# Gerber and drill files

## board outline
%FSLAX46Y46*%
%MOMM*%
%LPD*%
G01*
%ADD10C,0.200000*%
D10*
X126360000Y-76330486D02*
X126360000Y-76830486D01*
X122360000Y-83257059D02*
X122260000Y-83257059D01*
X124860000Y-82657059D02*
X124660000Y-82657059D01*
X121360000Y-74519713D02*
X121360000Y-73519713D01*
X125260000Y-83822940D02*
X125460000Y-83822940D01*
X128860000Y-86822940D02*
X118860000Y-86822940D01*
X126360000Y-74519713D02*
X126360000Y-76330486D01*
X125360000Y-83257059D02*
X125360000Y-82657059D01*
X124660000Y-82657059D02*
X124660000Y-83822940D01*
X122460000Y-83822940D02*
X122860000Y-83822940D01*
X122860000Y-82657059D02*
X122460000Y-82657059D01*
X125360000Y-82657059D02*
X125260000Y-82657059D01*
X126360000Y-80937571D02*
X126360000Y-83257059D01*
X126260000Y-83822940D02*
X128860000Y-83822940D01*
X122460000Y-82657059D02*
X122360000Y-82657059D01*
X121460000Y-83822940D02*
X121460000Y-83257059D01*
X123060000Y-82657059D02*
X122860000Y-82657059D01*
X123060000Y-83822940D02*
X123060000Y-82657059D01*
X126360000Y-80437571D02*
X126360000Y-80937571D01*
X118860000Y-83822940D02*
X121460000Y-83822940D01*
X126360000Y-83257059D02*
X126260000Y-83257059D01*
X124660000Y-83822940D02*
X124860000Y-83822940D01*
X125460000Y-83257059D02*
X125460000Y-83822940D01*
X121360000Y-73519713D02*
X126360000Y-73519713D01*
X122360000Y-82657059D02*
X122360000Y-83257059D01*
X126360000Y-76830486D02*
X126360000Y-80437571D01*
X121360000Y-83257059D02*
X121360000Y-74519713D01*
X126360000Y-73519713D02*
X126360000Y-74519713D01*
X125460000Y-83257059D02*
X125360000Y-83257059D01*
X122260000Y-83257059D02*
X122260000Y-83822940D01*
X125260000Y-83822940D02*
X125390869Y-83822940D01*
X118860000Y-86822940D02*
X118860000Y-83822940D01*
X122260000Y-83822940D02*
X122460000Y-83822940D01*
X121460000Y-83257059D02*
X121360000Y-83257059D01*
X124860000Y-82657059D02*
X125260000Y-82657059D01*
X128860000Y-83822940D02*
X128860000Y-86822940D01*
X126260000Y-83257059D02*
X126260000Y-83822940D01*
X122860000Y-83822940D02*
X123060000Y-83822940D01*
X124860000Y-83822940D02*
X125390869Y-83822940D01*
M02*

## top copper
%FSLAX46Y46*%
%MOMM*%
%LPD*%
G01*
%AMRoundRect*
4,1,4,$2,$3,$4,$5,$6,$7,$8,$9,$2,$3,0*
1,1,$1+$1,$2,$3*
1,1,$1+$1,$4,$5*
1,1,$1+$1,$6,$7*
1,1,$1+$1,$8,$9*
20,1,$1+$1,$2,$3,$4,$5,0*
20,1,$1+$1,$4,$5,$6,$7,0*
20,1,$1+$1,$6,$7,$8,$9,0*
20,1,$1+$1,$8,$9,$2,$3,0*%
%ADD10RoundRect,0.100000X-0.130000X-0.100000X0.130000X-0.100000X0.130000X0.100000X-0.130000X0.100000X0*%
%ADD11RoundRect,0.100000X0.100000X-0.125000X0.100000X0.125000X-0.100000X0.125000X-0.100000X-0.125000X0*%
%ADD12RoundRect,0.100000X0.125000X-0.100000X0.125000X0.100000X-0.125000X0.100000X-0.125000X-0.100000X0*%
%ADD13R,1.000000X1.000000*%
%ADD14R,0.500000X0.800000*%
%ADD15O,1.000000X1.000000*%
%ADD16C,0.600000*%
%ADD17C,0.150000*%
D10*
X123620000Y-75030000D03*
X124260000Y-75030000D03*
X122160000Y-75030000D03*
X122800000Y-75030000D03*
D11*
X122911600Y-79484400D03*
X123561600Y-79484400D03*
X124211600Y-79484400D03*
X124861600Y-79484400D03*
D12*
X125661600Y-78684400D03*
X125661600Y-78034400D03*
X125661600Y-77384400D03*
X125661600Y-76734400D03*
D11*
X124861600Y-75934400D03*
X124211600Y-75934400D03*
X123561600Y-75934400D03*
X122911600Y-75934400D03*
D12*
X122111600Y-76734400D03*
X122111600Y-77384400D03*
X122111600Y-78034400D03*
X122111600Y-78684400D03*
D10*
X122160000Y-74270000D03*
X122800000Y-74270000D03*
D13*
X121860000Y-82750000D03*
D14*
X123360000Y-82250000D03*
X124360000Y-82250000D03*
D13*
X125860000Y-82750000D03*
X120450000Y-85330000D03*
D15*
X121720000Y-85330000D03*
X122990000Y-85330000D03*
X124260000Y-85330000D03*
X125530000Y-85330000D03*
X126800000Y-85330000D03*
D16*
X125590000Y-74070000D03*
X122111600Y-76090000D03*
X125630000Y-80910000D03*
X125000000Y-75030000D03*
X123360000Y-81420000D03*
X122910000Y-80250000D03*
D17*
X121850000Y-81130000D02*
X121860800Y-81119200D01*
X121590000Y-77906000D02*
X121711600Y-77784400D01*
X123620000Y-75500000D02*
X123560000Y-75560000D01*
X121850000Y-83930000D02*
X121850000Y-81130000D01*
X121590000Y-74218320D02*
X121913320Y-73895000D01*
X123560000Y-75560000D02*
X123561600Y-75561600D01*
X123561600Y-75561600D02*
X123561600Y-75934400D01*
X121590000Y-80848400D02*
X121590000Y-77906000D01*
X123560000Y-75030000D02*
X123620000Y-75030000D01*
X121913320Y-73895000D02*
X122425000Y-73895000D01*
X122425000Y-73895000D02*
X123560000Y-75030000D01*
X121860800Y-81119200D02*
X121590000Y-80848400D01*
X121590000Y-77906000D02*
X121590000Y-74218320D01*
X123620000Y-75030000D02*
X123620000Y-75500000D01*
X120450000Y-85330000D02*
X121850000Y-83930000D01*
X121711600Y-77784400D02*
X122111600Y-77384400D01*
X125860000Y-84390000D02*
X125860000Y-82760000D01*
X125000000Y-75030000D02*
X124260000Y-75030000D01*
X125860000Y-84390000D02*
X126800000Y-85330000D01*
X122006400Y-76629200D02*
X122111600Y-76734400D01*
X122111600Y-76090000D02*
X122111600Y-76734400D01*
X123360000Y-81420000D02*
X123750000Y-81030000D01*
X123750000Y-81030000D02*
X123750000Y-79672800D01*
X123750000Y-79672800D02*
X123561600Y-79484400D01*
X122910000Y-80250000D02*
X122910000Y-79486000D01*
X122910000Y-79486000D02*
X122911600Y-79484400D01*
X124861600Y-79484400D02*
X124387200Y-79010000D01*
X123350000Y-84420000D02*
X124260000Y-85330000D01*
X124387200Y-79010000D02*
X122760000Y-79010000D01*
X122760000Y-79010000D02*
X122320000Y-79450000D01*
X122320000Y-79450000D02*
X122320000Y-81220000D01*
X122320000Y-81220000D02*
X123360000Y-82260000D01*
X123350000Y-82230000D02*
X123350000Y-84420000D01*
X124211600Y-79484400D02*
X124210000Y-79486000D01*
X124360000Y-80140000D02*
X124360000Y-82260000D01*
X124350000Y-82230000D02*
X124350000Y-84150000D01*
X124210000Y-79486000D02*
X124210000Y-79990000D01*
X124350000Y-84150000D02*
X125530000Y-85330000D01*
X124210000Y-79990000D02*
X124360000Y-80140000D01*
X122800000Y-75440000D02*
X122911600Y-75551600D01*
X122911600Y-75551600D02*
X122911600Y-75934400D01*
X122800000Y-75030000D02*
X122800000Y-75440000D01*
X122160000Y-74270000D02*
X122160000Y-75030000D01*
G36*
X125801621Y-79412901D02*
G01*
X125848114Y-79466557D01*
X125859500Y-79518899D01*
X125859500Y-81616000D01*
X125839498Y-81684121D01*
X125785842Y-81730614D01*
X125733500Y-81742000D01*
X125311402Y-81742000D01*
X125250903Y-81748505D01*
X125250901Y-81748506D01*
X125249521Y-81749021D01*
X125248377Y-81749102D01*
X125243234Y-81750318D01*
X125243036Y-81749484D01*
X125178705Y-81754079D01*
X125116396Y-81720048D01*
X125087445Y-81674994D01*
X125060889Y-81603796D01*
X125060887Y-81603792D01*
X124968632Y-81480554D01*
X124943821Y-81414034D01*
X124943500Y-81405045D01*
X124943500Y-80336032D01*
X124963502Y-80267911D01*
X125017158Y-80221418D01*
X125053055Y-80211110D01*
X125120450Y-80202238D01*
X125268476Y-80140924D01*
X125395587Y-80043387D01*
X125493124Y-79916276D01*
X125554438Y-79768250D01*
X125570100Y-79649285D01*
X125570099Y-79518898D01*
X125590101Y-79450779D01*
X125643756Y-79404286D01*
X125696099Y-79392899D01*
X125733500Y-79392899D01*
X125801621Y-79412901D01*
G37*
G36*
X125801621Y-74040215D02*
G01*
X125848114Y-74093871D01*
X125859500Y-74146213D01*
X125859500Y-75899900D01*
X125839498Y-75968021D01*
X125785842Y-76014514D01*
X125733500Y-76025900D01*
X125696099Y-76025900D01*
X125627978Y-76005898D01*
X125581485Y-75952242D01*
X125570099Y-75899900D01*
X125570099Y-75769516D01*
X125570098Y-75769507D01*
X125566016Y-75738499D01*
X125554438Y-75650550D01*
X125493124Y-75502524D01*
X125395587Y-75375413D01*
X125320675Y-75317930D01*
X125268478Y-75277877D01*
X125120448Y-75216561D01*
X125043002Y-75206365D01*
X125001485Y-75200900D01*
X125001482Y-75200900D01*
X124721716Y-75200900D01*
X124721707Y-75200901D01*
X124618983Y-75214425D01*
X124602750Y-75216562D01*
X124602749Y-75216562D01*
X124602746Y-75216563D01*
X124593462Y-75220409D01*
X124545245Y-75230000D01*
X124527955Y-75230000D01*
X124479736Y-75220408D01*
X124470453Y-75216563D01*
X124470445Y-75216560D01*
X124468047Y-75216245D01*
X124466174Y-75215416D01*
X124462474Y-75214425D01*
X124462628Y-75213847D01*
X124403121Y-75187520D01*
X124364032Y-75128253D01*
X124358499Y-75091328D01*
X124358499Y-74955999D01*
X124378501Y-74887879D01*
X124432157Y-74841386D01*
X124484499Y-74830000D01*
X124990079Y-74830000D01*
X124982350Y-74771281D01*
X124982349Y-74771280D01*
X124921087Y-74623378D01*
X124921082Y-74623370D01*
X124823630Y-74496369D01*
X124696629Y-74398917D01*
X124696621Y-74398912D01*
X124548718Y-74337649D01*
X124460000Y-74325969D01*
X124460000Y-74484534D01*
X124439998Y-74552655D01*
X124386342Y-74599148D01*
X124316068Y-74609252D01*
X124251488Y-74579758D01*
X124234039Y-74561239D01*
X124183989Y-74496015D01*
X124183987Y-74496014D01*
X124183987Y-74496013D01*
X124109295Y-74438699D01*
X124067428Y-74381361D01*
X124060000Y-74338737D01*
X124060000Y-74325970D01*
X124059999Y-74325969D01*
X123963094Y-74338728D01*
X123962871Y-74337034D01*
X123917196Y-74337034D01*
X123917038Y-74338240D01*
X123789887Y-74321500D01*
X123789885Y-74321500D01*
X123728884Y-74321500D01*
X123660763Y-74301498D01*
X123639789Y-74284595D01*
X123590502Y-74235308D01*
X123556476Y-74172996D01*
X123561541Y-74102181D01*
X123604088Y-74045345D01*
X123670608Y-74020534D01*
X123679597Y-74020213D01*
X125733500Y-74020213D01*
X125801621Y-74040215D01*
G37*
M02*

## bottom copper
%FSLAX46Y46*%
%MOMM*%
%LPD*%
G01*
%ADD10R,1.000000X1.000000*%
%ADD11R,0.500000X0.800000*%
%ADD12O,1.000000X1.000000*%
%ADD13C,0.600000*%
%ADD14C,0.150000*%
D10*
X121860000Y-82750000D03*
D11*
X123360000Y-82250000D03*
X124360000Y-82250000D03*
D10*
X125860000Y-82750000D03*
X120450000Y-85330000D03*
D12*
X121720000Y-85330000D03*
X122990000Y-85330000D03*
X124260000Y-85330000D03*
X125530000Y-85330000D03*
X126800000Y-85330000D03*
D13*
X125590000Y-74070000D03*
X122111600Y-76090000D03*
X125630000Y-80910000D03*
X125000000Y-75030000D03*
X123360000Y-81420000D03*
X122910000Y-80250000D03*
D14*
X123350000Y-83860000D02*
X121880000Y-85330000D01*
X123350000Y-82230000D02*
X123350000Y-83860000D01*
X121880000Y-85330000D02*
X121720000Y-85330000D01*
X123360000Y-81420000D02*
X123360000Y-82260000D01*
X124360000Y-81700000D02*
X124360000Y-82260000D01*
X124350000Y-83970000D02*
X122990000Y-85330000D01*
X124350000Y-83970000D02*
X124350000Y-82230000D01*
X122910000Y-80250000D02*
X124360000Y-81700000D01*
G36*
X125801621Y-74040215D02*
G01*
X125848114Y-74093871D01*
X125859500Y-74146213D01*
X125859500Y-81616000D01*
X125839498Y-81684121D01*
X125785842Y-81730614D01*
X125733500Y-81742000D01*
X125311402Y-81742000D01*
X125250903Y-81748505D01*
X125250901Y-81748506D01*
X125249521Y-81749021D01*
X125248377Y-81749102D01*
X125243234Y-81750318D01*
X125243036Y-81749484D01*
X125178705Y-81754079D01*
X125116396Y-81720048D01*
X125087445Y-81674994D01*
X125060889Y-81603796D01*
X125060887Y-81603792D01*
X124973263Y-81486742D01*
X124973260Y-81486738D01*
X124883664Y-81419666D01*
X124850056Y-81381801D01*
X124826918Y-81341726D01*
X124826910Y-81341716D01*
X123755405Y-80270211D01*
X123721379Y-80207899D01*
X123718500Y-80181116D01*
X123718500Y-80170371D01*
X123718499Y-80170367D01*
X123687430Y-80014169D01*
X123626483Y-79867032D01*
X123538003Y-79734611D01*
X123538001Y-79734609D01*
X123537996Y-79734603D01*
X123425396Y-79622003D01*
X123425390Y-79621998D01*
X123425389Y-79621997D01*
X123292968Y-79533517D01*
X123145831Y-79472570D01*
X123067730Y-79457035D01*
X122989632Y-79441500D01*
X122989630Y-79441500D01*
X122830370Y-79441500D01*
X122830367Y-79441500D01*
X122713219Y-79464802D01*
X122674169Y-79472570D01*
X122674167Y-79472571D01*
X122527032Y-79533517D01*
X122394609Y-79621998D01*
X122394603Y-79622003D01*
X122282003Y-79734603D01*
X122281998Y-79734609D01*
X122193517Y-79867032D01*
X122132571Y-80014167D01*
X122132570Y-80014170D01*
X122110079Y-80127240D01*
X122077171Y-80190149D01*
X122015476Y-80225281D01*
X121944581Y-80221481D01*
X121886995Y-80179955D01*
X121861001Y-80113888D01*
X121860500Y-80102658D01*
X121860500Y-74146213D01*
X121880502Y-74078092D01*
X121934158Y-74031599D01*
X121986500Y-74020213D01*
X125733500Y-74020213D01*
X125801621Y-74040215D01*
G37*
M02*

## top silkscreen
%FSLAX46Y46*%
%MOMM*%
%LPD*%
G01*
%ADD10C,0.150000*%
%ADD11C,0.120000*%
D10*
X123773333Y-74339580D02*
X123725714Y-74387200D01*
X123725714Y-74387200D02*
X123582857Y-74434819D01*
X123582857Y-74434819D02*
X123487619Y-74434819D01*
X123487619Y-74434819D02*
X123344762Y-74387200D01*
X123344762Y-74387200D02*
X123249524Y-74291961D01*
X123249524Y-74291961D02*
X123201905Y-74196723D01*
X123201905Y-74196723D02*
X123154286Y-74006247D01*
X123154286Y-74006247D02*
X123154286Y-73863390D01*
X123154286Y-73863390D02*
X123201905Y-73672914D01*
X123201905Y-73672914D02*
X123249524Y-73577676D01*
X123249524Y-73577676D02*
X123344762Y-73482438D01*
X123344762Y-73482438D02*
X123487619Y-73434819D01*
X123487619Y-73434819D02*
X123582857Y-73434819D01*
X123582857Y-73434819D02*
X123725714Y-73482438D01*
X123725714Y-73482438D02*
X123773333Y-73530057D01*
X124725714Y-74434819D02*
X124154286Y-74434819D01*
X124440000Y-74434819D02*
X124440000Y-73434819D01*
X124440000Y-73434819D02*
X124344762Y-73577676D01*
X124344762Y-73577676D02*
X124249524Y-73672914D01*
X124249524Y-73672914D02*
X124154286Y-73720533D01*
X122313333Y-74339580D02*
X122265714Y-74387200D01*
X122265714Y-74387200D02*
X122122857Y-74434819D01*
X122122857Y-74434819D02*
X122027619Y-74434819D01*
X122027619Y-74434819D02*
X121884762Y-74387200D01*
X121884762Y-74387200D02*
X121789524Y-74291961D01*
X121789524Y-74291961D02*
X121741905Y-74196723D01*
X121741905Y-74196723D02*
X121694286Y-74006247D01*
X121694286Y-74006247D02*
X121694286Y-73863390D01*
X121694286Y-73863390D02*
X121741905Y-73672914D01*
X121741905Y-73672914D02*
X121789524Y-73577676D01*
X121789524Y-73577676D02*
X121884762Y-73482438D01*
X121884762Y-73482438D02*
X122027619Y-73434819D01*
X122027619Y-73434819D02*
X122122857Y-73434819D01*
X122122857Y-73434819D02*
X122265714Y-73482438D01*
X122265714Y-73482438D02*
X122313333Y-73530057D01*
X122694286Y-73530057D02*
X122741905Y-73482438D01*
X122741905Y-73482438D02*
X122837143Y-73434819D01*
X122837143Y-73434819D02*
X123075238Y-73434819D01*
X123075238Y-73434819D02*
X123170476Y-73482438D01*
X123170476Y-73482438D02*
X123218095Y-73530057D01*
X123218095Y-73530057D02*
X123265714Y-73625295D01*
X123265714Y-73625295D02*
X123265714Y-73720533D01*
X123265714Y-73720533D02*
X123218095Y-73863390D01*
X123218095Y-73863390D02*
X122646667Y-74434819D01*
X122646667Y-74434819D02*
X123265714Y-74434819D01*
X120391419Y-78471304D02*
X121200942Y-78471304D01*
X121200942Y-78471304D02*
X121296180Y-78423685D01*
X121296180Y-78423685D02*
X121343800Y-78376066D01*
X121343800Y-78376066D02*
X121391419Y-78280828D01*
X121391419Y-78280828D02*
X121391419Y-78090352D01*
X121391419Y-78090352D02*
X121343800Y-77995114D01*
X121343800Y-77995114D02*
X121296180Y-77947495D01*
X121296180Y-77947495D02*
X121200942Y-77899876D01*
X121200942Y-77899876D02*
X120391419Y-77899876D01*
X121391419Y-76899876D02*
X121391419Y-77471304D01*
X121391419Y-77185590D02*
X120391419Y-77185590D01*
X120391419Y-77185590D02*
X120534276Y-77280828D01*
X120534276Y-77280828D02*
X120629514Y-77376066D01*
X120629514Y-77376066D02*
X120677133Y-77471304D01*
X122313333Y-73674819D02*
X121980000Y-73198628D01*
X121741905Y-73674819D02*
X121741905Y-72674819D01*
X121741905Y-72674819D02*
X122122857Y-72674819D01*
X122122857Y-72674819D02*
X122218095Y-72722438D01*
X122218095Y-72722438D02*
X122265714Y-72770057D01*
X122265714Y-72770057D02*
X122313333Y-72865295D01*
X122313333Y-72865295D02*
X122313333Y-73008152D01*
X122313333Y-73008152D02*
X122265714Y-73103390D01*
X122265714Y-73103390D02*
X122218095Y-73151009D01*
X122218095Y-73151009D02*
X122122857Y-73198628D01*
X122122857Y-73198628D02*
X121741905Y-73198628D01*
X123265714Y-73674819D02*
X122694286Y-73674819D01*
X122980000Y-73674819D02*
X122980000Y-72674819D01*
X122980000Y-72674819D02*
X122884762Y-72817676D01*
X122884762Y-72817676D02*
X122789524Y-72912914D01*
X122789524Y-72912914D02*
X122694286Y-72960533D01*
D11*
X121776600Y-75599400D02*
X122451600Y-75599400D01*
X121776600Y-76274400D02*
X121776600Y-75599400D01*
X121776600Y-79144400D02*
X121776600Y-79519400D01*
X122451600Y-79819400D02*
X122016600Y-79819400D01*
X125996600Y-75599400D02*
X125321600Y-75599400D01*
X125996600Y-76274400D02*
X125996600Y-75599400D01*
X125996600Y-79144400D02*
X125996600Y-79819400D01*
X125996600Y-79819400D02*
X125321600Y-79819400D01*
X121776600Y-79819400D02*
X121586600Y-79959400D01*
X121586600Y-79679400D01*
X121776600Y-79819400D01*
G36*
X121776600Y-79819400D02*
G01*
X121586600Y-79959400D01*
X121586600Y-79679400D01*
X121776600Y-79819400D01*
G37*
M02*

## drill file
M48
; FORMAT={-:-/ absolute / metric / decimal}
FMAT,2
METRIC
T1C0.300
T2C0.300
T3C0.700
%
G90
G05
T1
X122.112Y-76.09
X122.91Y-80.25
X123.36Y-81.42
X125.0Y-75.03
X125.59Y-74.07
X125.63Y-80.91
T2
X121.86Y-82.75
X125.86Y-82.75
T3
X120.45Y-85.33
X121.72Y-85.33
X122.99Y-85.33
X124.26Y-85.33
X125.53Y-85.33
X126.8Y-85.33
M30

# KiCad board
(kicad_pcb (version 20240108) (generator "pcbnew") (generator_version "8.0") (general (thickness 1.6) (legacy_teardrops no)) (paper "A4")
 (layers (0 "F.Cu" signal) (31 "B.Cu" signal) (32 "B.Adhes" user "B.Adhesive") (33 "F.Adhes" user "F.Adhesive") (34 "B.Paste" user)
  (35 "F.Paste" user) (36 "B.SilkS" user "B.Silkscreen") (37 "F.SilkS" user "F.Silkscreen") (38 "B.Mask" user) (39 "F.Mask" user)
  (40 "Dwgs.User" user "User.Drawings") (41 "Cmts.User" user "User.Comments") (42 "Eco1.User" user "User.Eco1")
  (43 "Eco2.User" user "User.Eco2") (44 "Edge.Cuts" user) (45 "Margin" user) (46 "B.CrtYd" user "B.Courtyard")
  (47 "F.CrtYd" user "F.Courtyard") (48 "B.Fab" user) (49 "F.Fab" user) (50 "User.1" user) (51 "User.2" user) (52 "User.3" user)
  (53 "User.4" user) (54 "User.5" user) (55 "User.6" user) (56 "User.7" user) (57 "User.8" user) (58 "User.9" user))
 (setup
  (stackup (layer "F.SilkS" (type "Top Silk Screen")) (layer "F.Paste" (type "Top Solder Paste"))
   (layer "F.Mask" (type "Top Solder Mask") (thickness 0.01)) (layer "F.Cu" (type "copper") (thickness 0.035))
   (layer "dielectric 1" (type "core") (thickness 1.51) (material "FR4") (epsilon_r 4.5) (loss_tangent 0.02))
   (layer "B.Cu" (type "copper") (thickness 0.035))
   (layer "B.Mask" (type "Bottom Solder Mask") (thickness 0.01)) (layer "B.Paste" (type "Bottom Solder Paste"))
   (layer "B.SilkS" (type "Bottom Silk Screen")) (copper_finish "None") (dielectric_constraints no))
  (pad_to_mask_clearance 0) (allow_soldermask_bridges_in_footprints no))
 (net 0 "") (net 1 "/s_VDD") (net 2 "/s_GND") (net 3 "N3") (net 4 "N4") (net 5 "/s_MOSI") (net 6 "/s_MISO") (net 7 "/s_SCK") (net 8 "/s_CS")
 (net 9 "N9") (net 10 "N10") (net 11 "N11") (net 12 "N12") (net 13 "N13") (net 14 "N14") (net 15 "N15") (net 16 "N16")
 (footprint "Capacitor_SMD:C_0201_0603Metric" (layer "F.Cu") (at 123.94 75.03)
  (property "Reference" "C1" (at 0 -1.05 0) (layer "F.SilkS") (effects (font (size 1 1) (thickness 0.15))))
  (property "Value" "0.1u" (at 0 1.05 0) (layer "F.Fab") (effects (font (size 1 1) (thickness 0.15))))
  (pad "" smd roundrect (at -0.345 0) (size 0.318 0.36) (layers "F.Paste") (roundrect_rratio 0.25))
  (pad "" smd roundrect (at 0.345 0) (size 0.318 0.36) (layers "F.Paste") (roundrect_rratio 0.25))
  (pad "1" smd roundrect (at -0.32 0) (size 0.46 0.4) (layers "F.Cu" "F.Mask") (roundrect_rratio 0.25) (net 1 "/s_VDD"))
  (pad "2" smd roundrect (at 0.32 0) (size 0.46 0.4) (layers "F.Cu" "F.Mask") (roundrect_rratio 0.25) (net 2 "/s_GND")))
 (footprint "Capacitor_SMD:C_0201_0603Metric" (layer "F.Cu") (at 122.48 75.03)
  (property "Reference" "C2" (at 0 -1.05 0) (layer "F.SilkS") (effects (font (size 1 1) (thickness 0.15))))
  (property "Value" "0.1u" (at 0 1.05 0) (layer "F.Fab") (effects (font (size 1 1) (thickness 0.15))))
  (pad "" smd roundrect (at -0.345 0) (size 0.318 0.36) (layers "F.Paste") (roundrect_rratio 0.25))
  (pad "" smd roundrect (at 0.345 0) (size 0.318 0.36) (layers "F.Paste") (roundrect_rratio 0.25))
  (pad "1" smd roundrect (at -0.32 0) (size 0.46 0.4) (layers "F.Cu" "F.Mask") (roundrect_rratio 0.25) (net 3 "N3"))
  (pad "2" smd roundrect (at 0.32 0) (size 0.46 0.4) (layers "F.Cu" "F.Mask") (roundrect_rratio 0.25) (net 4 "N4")))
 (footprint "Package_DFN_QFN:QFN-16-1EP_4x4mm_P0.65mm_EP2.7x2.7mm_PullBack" (layer "F.Cu") (at 123.8866 77.7094 90)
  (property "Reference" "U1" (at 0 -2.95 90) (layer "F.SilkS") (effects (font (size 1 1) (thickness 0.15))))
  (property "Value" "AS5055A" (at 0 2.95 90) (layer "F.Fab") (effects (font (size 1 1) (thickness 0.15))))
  (fp_line (start 2.11 -2.11) (end 2.11 -1.435) (stroke (width 0.12) (type solid)) (layer "F.SilkS"))
  (fp_line (start 1.435 -2.11) (end 2.11 -2.11) (stroke (width 0.12) (type solid)) (layer "F.SilkS"))
  (fp_line (start -1.435 -2.11) (end -1.81 -2.11) (stroke (width 0.12) (type solid)) (layer "F.SilkS"))
  (fp_line (start -2.11 -1.435) (end -2.11 -1.87) (stroke (width 0.12) (type solid)) (layer "F.SilkS"))
  (fp_line (start 2.11 2.11) (end 2.11 1.435) (stroke (width 0.12) (type solid)) (layer "F.SilkS"))
  (fp_line (start 1.435 2.11) (end 2.11 2.11) (stroke (width 0.12) (type solid)) (layer "F.SilkS"))
  (fp_line (start -1.435 2.11) (end -2.11 2.11) (stroke (width 0.12) (type solid)) (layer "F.SilkS"))
  (fp_line (start -2.11 2.11) (end -2.11 1.435) (stroke (width 0.12) (type solid)) (layer "F.SilkS"))
  (fp_poly
   (pts (xy -2.11 -2.11) (xy -2.25 -2.3) (xy -1.97 -2.3) (xy -2.11 -2.11)) (stroke (width 0.12) (type solid)) (fill solid) (layer "F.SilkS"))
  (pad "1" smd roundrect (at -1.775 -0.975 90) (size 0.45 0.4) (layers "F.Cu" "F.Paste" "F.Mask") (roundrect_rratio 0.25) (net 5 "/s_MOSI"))
  (pad "2" smd roundrect (at -1.775 -0.325 90) (size 0.45 0.4) (layers "F.Cu" "F.Paste" "F.Mask") (roundrect_rratio 0.25) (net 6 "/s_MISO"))
  (pad "3" smd roundrect (at -1.775 0.325 90) (size 0.45 0.4) (layers "F.Cu" "F.Paste" "F.Mask") (roundrect_rratio 0.25) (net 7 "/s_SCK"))
  (pad "4" smd roundrect (at -1.775 0.975 90) (size 0.45 0.4) (layers "F.Cu" "F.Paste" "F.Mask") (roundrect_rratio 0.25) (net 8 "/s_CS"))
  (pad "5" smd roundrect (at -0.975 1.775 90) (size 0.4 0.45) (layers "F.Cu" "F.Paste" "F.Mask") (roundrect_rratio 0.25) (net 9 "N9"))
  (pad "6" smd roundrect (at -0.325 1.775 90) (size 0.4 0.45) (layers "F.Cu" "F.Paste" "F.Mask") (roundrect_rratio 0.25) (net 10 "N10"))
  (pad "7" smd roundrect (at 0.325 1.775 90) (size 0.4 0.45) (layers "F.Cu" "F.Paste" "F.Mask") (roundrect_rratio 0.25) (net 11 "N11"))
  (pad "8" smd roundrect (at 0.975 1.775 90) (size 0.4 0.45) (layers "F.Cu" "F.Paste" "F.Mask") (roundrect_rratio 0.25) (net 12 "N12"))
  (pad "9" smd roundrect (at 1.775 0.975 90) (size 0.45 0.4) (layers "F.Cu" "F.Paste" "F.Mask") (roundrect_rratio 0.25) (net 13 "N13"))
  (pad "10" smd roundrect (at 1.775 0.325 90) (size 0.45 0.4) (layers "F.Cu" "F.Paste" "F.Mask") (roundrect_rratio 0.25) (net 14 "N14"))
  (pad "11" smd roundrect (at 1.775 -0.325 90) (size 0.45 0.4) (layers "F.Cu" "F.Paste" "F.Mask") (roundrect_rratio 0.25) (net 1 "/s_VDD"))
  (pad "12" smd roundrect (at 1.775 -0.975 90) (size 0.45 0.4) (layers "F.Cu" "F.Paste" "F.Mask") (roundrect_rratio 0.25) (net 4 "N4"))
  (pad "13" smd roundrect (at 0.975 -1.775 90) (size 0.4 0.45) (layers "F.Cu" "F.Paste" "F.Mask") (roundrect_rratio 0.25) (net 2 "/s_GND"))
  (pad "14" smd roundrect (at 0.325 -1.775 90) (size 0.4 0.45) (layers "F.Cu" "F.Paste" "F.Mask") (roundrect_rratio 0.25) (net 1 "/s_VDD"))
  (pad "15" smd roundrect (at -0.325 -1.775 90) (size 0.4 0.45) (layers "F.Cu" "F.Paste" "F.Mask") (roundrect_rratio 0.25) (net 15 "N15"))
  (pad "16" smd roundrect (at -0.975 -1.775 90) (size 0.4 0.45) (layers "F.Cu" "F.Paste" "F.Mask") (roundrect_rratio 0.25) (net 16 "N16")))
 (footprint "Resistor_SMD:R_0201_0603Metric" (layer "F.Cu") (at 122.48 74.27)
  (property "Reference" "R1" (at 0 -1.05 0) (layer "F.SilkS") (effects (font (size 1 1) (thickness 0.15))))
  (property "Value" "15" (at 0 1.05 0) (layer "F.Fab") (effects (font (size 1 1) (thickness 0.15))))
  (pad "" smd roundrect (at -0.345 0) (size 0.318 0.36) (layers "F.Paste") (roundrect_rratio 0.25))
  (pad "" smd roundrect (at 0.345 0) (size 0.318 0.36) (layers "F.Paste") (roundrect_rratio 0.25))
  (pad "1" smd roundrect (at -0.32 0) (size 0.46 0.4) (layers "F.Cu" "F.Mask") (roundrect_rratio 0.25) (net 3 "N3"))
  (pad "2" smd roundrect (at 0.32 0) (size 0.46 0.4) (layers "F.Cu" "F.Mask") (roundrect_rratio 0.25) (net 1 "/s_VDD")))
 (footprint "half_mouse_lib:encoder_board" (layer "B.Cu") (at 121.86 82.75 -90)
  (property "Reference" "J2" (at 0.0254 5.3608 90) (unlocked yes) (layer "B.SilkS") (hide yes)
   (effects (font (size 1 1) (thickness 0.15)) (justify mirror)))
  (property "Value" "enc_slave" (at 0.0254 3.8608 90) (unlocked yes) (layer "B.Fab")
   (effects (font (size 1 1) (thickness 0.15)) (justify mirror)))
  (pad "1" thru_hole rect (at 0 0 270) (size 1 1) (drill 0.3) (layers "*.Cu" "*.Mask") (remove_unused_layers no) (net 1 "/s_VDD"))
  (pad "2" smd rect (at -0.5 -1.5 270) (size 0.8 0.5) (layers "B.Cu" "B.Paste" "B.Mask") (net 6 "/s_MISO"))
  (pad "3" smd rect (at -0.5 -2.5 270) (size 0.8 0.5) (layers "B.Cu" "B.Paste" "B.Mask" "Eco1.User") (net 5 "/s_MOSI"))
  (pad "4" smd rect (at -0.5 -1.5 270) (size 0.8 0.5) (layers "F.Cu" "F.Paste" "F.Mask") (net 8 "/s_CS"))
  (pad "5" smd rect (at -0.5 -2.5 270) (size 0.8 0.5) (layers "F.Cu" "F.Paste" "F.Mask") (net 7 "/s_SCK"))
  (pad "6" thru_hole rect (at 0 -4 270) (size 1 1) (drill 0.3) (layers "*.Cu" "*.Mask") (remove_unused_layers no) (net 2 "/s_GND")))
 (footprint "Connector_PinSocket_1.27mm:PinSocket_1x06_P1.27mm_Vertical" (layer "B.Cu") (at 120.45 85.33 -90)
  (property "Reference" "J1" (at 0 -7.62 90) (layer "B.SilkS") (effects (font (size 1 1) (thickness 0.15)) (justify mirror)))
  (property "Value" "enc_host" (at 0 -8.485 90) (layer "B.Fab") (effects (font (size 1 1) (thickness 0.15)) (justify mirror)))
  (pad "1" thru_hole rect (at 0 0 270) (size 1 1) (drill 0.7) (layers "*.Cu" "*.Mask") (remove_unused_layers no) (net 1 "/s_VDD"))
  (pad "2" thru_hole oval (at 0 -1.27 270) (size 1 1) (drill 0.7) (layers "*.Cu" "*.Mask") (remove_unused_layers no) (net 6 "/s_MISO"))
  (pad "3" thru_hole oval (at 0 -2.54 270) (size 1 1) (drill 0.7) (layers "*.Cu" "*.Mask") (remove_unused_layers no) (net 5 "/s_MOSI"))
  (pad "4" thru_hole oval (at 0 -3.81 270) (size 1 1) (drill 0.7) (layers "*.Cu" "*.Mask") (remove_unused_layers no) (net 8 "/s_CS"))
  (pad "5" thru_hole oval (at 0 -5.08 270) (size 1 1) (drill 0.7) (layers "*.Cu" "*.Mask") (remove_unused_layers no) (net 7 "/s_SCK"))
  (pad "6" thru_hole oval (at 0 -6.35 270) (size 1 1) (drill 0.7) (layers "*.Cu" "*.Mask") (remove_unused_layers no) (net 2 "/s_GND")))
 (gr_line (start 126.36 76.330486) (end 126.36 76.830486) (stroke (width 0.2) (type default)) (layer "Edge.Cuts"))
 (gr_line (start 122.36 83.257059) (end 122.26 83.257059) (stroke (width 0.2) (type default)) (layer "Edge.Cuts"))
 (gr_line (start 124.86 82.657059) (end 124.66 82.657059) (stroke (width 0.2) (type default)) (layer "Edge.Cuts"))
 (gr_line (start 121.36 74.519713) (end 121.36 73.519713) (stroke (width 0.2) (type default)) (layer "Edge.Cuts"))
 (gr_line (start 125.26 83.82294) (end 125.46 83.82294) (stroke (width 0.2) (type default)) (layer "Edge.Cuts"))
 (gr_line (start 128.86 86.82294) (end 118.86 86.82294) (stroke (width 0.2) (type default)) (layer "Edge.Cuts"))
 (gr_line (start 126.36 74.519713) (end 126.36 76.330486) (stroke (width 0.2) (type default)) (layer "Edge.Cuts"))
 (gr_line (start 125.36 83.257059) (end 125.36 82.657059) (stroke (width 0.2) (type default)) (layer "Edge.Cuts"))
 (gr_line (start 124.66 82.657059) (end 124.66 83.82294) (stroke (width 0.2) (type default)) (layer "Edge.Cuts"))
 (gr_line (start 122.46 83.82294) (end 122.86 83.82294) (stroke (width 0.2) (type default)) (layer "Edge.Cuts"))
 (gr_line (start 122.86 82.657059) (end 122.46 82.657059) (stroke (width 0.2) (type default)) (layer "Edge.Cuts"))
 (gr_line (start 125.36 82.657059) (end 125.26 82.657059) (stroke (width 0.2) (type default)) (layer "Edge.Cuts"))
 (gr_line (start 126.36 80.937571) (end 126.36 83.257059) (stroke (width 0.2) (type default)) (layer "Edge.Cuts"))
 (gr_line (start 126.26 83.82294) (end 128.86 83.82294) (stroke (width 0.2) (type default)) (layer "Edge.Cuts"))
 (gr_line (start 122.46 82.657059) (end 122.36 82.657059) (stroke (width 0.2) (type default)) (layer "Edge.Cuts"))
 (gr_line (start 121.46 83.82294) (end 121.46 83.257059) (stroke (width 0.2) (type default)) (layer "Edge.Cuts"))
 (gr_line (start 123.06 82.657059) (end 122.86 82.657059) (stroke (width 0.2) (type default)) (layer "Edge.Cuts"))
 (gr_line (start 123.06 83.82294) (end 123.06 82.657059) (stroke (width 0.2) (type default)) (layer "Edge.Cuts"))
 (gr_line (start 126.36 80.437571) (end 126.36 80.937571) (stroke (width 0.2) (type default)) (layer "Edge.Cuts"))
 (gr_line (start 118.86 83.82294) (end 121.46 83.82294) (stroke (width 0.2) (type default)) (layer "Edge.Cuts"))
 (gr_line (start 126.36 83.257059) (end 126.26 83.257059) (stroke (width 0.2) (type default)) (layer "Edge.Cuts"))
 (gr_line (start 124.66 83.82294) (end 124.86 83.82294) (stroke (width 0.2) (type default)) (layer "Edge.Cuts"))
 (gr_line (start 125.46 83.257059) (end 125.46 83.82294) (stroke (width 0.2) (type default)) (layer "Edge.Cuts"))
 (gr_line (start 121.36 73.519713) (end 126.36 73.519713) (stroke (width 0.2) (type default)) (layer "Edge.Cuts"))
 (gr_line (start 122.36 82.657059) (end 122.36 83.257059) (stroke (width 0.2) (type default)) (layer "Edge.Cuts"))
 (gr_line (start 126.36 76.830486) (end 126.36 80.437571) (stroke (width 0.2) (type default)) (layer "Edge.Cuts"))
 (gr_line (start 121.36 83.257059) (end 121.36 74.519713) (stroke (width 0.2) (type default)) (layer "Edge.Cuts"))
 (gr_line (start 126.36 73.519713) (end 126.36 74.519713) (stroke (width 0.2) (type default)) (layer "Edge.Cuts"))
 (gr_line (start 125.46 83.257059) (end 125.36 83.257059) (stroke (width 0.2) (type default)) (layer "Edge.Cuts"))
 (gr_line (start 122.26 83.257059) (end 122.26 83.82294) (stroke (width 0.2) (type default)) (layer "Edge.Cuts"))
 (gr_line (start 125.26 83.82294) (end 125.390869 83.82294) (stroke (width 0.2) (type default)) (layer "Edge.Cuts"))
 (gr_line (start 118.86 86.82294) (end 118.86 83.82294) (stroke (width 0.2) (type default)) (layer "Edge.Cuts"))
 (gr_line (start 122.26 83.82294) (end 122.46 83.82294) (stroke (width 0.2) (type default)) (layer "Edge.Cuts"))
 (gr_line (start 121.46 83.257059) (end 121.36 83.257059) (stroke (width 0.2) (type default)) (layer "Edge.Cuts"))
 (gr_line (start 124.86 82.657059) (end 125.26 82.657059) (stroke (width 0.2) (type default)) (layer "Edge.Cuts"))
 (gr_line (start 128.86 83.82294) (end 128.86 86.82294) (stroke (width 0.2) (type default)) (layer "Edge.Cuts"))
 (gr_line (start 126.26 83.257059) (end 126.26 83.82294) (stroke (width 0.2) (type default)) (layer "Edge.Cuts"))
 (gr_line (start 122.86 83.82294) (end 123.06 83.82294) (stroke (width 0.2) (type default)) (layer "Edge.Cuts"))
 (gr_line (start 124.86 83.82294) (end 125.390869 83.82294) (stroke (width 0.2) (type default)) (layer "Edge.Cuts"))
 (segment (start 121.85 81.13) (end 121.8608 81.1192) (width 0.15) (layer "F.Cu") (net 1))
 (segment (start 121.59 77.906) (end 121.7116 77.7844) (width 0.15) (layer "F.Cu") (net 1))
 (segment (start 123.62 75.5) (end 123.56 75.56) (width 0.15) (layer "F.Cu") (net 1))
 (segment (start 121.85 83.93) (end 121.85 81.13) (width 0.15) (layer "F.Cu") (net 1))
 (segment (start 121.59 74.21832) (end 121.91332 73.895) (width 0.15) (layer "F.Cu") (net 1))
 (segment (start 123.56 75.56) (end 123.5616 75.5616) (width 0.15) (layer "F.Cu") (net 1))
 (segment (start 123.5616 75.5616) (end 123.5616 75.9344) (width 0.15) (layer "F.Cu") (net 1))
 (segment (start 121.59 80.8484) (end 121.59 77.906) (width 0.15) (layer "F.Cu") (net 1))
 (segment (start 123.56 75.03) (end 123.62 75.03) (width 0.15) (layer "F.Cu") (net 1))
 (segment (start 121.91332 73.895) (end 122.425 73.895) (width 0.15) (layer "F.Cu") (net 1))
 (segment (start 122.425 73.895) (end 123.56 75.03) (width 0.15) (layer "F.Cu") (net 1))
 (segment (start 121.8608 81.1192) (end 121.59 80.8484) (width 0.15) (layer "F.Cu") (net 1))
 (segment (start 121.59 77.906) (end 121.59 74.21832) (width 0.15) (layer "F.Cu") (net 1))
 (segment (start 123.62 75.03) (end 123.62 75.5) (width 0.15) (layer "F.Cu") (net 1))
 (segment (start 120.45 85.33) (end 121.85 83.93) (width 0.15) (layer "F.Cu") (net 1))
 (segment (start 121.7116 77.7844) (end 122.1116 77.3844) (width 0.15) (layer "F.Cu") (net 1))
 (segment (start 125.86 84.39) (end 125.86 82.76) (width 0.15) (layer "F.Cu") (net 2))
 (segment (start 125 75.03) (end 124.26 75.03) (width 0.15) (layer "F.Cu") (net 2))
 (segment (start 125.86 84.39) (end 126.8 85.33) (width 0.15) (layer "F.Cu") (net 2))
 (segment (start 122.0064 76.6292) (end 122.1116 76.7344) (width 0.15) (layer "F.Cu") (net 2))
 (segment (start 122.1116 76.09) (end 122.1116 76.7344) (width 0.15) (layer "F.Cu") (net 2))
 (via (at 125.59 74.07) (size 0.6) (drill 0.3) (layers "F.Cu" "B.Cu") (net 2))
 (via (at 122.1116 76.09) (size 0.6) (drill 0.3) (layers "F.Cu" "B.Cu") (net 2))
 (via (at 125.63 80.91) (size 0.6) (drill 0.3) (layers "F.Cu" "B.Cu") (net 2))
 (via (at 125 75.03) (size 0.6) (drill 0.3) (layers "F.Cu" "B.Cu") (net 2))
 (segment (start 123.36 81.42) (end 123.75 81.03) (width 0.15) (layer "F.Cu") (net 6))
 (segment (start 123.75 81.03) (end 123.75 79.6728) (width 0.15) (layer "F.Cu") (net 6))
 (segment (start 123.75 79.6728) (end 123.5616 79.4844) (width 0.15) (layer "F.Cu") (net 6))
 (via (at 123.36 81.42) (size 0.6) (drill 0.3) (layers "F.Cu" "B.Cu") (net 6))
 (segment (start 123.35 83.86) (end 121.88 85.33) (width 0.15) (layer "B.Cu") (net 6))
 (segment (start 123.35 82.23) (end 123.35 83.86) (width 0.15) (layer "B.Cu") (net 6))
 (segment (start 121.88 85.33) (end 121.72 85.33) (width 0.15) (layer "B.Cu") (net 6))
 (segment (start 123.36 81.42) (end 123.36 82.26) (width 0.15) (layer "B.Cu") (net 6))
 (segment (start 122.91 80.25) (end 122.91 79.486) (width 0.15) (layer "F.Cu") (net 5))
 (segment (start 122.91 79.486) (end 122.9116 79.4844) (width 0.15) (layer "F.Cu") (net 5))
 (via (at 122.91 80.25) (size 0.6) (drill 0.3) (layers "F.Cu" "B.Cu") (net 5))
 (segment (start 124.36 81.7) (end 124.36 82.26) (width 0.15) (layer "B.Cu") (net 5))
 (segment (start 124.35 83.97) (end 122.99 85.33) (width 0.15) (layer "B.Cu") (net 5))
 (segment (start 124.35 83.97) (end 124.35 82.23) (width 0.15) (layer "B.Cu") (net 5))
 (segment (start 122.91 80.25) (end 124.36 81.7) (width 0.15) (layer "B.Cu") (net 5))
 (segment (start 124.8616 79.4844) (end 124.3872 79.01) (width 0.15) (layer "F.Cu") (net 8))
 (segment (start 123.35 84.42) (end 124.26 85.33) (width 0.15) (layer "F.Cu") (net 8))
 (segment (start 124.3872 79.01) (end 122.76 79.01) (width 0.15) (layer "F.Cu") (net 8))
 (segment (start 122.76 79.01) (end 122.32 79.45) (width 0.15) (layer "F.Cu") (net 8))
 (segment (start 122.32 79.45) (end 122.32 81.22) (width 0.15) (layer "F.Cu") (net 8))
 (segment (start 122.32 81.22) (end 123.36 82.26) (width 0.15) (layer "F.Cu") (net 8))
 (segment (start 123.35 82.23) (end 123.35 84.42) (width 0.15) (layer "F.Cu") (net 8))
 (segment (start 124.2116 79.4844) (end 124.21 79.486) (width 0.15) (layer "F.Cu") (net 7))
 (segment (start 124.36 80.14) (end 124.36 82.26) (width 0.15) (layer "F.Cu") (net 7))
 (segment (start 124.35 82.23) (end 124.35 84.15) (width 0.15) (layer "F.Cu") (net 7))
 (segment (start 124.21 79.486) (end 124.21 79.99) (width 0.15) (layer "F.Cu") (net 7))
 (segment (start 124.35 84.15) (end 125.53 85.33) (width 0.15) (layer "F.Cu") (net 7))
 (segment (start 124.21 79.99) (end 124.36 80.14) (width 0.15) (layer "F.Cu") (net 7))
 (segment (start 122.8 75.44) (end 122.9116 75.5516) (width 0.15) (layer "F.Cu") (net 4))
 (segment (start 122.9116 75.5516) (end 122.9116 75.9344) (width 0.15) (layer "F.Cu") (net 4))
 (segment (start 122.8 75.03) (end 122.8 75.44) (width 0.15) (layer "F.Cu") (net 4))
 (segment (start 122.16 74.27) (end 122.16 75.03) (width 0.15) (layer "F.Cu") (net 3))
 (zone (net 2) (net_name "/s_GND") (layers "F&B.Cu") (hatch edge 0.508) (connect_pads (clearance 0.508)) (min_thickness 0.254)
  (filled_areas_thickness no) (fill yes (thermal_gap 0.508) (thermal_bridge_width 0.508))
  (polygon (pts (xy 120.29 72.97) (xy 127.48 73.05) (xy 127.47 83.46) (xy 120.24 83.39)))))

